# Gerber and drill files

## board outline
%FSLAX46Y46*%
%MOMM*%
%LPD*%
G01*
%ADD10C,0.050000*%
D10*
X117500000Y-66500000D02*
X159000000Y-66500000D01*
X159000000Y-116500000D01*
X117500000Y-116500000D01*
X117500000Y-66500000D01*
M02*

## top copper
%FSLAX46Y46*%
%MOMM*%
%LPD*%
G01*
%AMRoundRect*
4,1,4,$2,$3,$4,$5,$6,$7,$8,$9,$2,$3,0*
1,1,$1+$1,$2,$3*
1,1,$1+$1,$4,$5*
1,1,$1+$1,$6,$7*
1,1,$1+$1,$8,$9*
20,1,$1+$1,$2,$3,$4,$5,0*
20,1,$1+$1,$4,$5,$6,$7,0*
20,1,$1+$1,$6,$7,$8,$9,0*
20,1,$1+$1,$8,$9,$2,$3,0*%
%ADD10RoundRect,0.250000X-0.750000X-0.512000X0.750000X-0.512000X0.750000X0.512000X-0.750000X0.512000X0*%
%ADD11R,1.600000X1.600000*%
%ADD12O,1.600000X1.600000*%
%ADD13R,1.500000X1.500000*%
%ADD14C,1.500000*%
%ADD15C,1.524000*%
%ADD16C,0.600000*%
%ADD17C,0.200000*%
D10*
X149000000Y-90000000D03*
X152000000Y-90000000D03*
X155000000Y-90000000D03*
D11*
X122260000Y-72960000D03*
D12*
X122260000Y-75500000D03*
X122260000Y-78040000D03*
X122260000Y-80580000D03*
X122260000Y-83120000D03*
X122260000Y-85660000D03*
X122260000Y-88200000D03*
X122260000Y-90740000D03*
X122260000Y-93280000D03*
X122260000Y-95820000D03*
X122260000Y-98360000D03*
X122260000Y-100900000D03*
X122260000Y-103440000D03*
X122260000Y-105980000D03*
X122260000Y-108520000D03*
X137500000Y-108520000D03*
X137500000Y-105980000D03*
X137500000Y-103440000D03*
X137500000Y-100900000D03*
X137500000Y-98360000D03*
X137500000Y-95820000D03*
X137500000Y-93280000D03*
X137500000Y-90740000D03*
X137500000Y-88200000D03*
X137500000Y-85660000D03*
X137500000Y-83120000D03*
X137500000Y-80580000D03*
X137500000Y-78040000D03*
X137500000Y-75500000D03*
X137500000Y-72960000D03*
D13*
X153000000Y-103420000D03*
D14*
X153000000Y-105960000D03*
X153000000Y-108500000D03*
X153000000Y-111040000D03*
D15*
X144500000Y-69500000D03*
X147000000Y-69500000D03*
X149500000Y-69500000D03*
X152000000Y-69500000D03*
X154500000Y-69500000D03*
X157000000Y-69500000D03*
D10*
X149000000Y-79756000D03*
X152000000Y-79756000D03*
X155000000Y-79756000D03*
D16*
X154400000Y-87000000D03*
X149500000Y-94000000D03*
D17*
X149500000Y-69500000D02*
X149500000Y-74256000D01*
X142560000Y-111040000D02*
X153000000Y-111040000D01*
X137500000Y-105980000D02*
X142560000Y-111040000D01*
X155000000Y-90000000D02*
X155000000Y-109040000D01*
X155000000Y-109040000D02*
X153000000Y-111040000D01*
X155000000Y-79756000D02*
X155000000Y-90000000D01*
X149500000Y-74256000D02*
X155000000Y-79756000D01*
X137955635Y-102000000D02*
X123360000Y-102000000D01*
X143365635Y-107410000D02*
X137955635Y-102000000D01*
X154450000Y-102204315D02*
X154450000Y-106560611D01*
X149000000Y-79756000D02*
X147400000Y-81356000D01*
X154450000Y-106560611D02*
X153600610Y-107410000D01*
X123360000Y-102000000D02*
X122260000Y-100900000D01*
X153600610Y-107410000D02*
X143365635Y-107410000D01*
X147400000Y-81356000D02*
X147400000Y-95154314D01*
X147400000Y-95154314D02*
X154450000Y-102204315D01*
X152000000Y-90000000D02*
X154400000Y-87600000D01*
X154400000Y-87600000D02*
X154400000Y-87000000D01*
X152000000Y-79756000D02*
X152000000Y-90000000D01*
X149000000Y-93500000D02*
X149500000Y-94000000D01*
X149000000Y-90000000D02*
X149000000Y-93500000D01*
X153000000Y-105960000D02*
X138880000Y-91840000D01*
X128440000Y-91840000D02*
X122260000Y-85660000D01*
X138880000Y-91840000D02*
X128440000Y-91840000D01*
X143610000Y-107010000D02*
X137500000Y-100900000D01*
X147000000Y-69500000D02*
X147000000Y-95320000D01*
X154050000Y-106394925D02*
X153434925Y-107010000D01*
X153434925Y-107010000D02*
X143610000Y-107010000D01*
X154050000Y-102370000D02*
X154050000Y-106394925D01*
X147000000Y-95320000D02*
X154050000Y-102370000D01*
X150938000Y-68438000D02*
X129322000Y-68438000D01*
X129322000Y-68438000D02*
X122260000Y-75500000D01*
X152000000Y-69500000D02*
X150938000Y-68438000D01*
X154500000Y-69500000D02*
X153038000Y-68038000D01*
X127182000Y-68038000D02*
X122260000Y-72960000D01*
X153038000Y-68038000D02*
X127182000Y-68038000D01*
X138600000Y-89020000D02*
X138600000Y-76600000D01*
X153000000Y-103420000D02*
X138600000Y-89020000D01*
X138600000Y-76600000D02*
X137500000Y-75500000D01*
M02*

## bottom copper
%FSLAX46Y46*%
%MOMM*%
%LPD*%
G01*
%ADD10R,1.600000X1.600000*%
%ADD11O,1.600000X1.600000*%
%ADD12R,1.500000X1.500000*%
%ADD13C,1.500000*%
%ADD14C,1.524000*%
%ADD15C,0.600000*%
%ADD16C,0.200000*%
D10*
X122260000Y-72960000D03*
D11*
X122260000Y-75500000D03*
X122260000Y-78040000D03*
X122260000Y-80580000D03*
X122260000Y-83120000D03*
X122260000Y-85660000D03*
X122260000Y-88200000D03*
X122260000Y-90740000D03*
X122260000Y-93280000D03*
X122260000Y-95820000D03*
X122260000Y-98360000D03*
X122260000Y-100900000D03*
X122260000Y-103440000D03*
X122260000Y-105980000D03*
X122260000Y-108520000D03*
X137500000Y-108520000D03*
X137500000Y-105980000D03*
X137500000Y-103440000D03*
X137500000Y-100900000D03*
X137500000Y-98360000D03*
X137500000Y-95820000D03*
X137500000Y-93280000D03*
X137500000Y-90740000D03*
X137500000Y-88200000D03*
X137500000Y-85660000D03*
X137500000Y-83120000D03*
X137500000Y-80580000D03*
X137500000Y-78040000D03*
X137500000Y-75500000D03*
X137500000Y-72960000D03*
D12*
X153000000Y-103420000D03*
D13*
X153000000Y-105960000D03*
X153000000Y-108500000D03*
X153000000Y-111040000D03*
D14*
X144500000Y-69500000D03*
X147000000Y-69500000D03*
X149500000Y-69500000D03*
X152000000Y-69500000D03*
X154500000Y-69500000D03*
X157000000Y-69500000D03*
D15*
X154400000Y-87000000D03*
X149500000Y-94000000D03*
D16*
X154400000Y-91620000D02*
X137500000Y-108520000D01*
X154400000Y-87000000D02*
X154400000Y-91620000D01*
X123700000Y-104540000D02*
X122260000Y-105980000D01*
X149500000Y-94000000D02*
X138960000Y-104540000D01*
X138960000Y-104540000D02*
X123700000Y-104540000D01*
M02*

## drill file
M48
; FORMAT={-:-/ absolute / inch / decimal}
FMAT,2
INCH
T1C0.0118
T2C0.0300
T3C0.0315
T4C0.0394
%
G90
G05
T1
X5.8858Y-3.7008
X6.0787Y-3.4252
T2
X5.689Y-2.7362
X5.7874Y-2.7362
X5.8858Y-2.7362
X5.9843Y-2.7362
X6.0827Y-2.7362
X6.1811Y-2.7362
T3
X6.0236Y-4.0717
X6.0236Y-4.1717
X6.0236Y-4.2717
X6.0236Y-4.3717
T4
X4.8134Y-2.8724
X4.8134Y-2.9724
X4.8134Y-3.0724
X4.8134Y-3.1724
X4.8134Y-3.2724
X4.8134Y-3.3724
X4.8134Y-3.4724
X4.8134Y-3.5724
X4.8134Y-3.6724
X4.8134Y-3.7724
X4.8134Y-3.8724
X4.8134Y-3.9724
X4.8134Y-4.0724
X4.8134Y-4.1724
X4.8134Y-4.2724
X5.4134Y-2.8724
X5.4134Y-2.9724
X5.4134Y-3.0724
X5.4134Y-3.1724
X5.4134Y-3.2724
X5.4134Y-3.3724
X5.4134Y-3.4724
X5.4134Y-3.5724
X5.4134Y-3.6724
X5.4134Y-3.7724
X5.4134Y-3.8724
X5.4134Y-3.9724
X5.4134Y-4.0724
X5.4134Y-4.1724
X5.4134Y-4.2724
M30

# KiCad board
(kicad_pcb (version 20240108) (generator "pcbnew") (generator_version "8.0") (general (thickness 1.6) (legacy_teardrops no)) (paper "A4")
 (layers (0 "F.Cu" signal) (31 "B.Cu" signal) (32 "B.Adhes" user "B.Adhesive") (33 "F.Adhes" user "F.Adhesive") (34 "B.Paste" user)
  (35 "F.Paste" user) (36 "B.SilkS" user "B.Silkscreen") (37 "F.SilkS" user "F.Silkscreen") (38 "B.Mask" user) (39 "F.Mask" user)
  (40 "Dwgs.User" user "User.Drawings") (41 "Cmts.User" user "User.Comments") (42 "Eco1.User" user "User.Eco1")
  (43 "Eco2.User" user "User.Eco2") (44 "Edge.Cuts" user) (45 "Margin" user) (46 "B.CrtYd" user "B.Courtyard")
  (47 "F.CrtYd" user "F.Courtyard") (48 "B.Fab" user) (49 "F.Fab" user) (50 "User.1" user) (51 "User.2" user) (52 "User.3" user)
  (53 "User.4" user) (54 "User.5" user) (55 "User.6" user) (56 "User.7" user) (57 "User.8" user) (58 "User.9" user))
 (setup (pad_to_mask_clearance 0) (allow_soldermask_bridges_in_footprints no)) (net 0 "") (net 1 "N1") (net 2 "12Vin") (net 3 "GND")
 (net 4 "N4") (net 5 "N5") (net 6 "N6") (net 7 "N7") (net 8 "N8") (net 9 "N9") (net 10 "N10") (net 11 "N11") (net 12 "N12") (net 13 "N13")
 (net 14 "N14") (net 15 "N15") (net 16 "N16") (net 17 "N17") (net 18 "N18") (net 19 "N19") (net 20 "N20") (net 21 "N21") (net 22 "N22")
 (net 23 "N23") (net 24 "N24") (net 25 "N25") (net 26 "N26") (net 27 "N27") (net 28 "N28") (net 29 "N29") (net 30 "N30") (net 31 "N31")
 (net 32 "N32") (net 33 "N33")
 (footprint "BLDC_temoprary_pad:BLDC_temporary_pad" (layer "F.Cu") (at 152 95)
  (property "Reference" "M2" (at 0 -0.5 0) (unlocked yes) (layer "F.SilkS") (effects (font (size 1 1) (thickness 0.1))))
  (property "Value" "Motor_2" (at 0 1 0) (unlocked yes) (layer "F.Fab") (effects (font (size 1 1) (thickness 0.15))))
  (pad "1" smd roundrect (at -3 -5) (size 2 1.524) (layers "F.Cu" "F.Paste" "F.Mask") (roundrect_rratio 0.1640419948) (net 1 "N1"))
  (pad "2" smd roundrect (at 0 -5) (size 2 1.524) (layers "F.Cu" "F.Paste" "F.Mask") (roundrect_rratio 0.1640419948) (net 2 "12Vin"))
  (pad "3" smd roundrect (at 3 -5) (size 2 1.524) (layers "F.Cu" "F.Paste" "F.Mask") (roundrect_rratio 0.1640419948) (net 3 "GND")))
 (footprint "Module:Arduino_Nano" (layer "F.Cu") (at 122.26 72.96)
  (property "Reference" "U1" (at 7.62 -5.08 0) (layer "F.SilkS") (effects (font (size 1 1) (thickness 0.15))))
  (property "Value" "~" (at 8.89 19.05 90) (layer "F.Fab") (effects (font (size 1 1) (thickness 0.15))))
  (pad "1" thru_hole rect (at 0 0) (size 1.6 1.6) (drill 1) (layers "*.Cu" "*.Mask") (remove_unused_layers no) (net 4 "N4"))
  (pad "2" thru_hole oval (at 0 2.54) (size 1.6 1.6) (drill 1) (layers "*.Cu" "*.Mask") (remove_unused_layers no) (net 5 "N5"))
  (pad "3" thru_hole oval (at 0 5.08) (size 1.6 1.6) (drill 1) (layers "*.Cu" "*.Mask") (remove_unused_layers no) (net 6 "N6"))
  (pad "4" thru_hole oval (at 0 7.62) (size 1.6 1.6) (drill 1) (layers "*.Cu" "*.Mask") (remove_unused_layers no) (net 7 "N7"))
  (pad "5" thru_hole oval (at 0 10.16) (size 1.6 1.6) (drill 1) (layers "*.Cu" "*.Mask") (remove_unused_layers no) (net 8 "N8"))
  (pad "6" thru_hole oval (at 0 12.7) (size 1.6 1.6) (drill 1) (layers "*.Cu" "*.Mask") (remove_unused_layers no) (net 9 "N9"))
  (pad "7" thru_hole oval (at 0 15.24) (size 1.6 1.6) (drill 1) (layers "*.Cu" "*.Mask") (remove_unused_layers no) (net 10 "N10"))
  (pad "8" thru_hole oval (at 0 17.78) (size 1.6 1.6) (drill 1) (layers "*.Cu" "*.Mask") (remove_unused_layers no) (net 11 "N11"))
  (pad "9" thru_hole oval (at 0 20.32) (size 1.6 1.6) (drill 1) (layers "*.Cu" "*.Mask") (remove_unused_layers no) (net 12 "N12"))
  (pad "10" thru_hole oval (at 0 22.86) (size 1.6 1.6) (drill 1) (layers "*.Cu" "*.Mask") (remove_unused_layers no) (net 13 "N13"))
  (pad "11" thru_hole oval (at 0 25.4) (size 1.6 1.6) (drill 1) (layers "*.Cu" "*.Mask") (remove_unused_layers no) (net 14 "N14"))
  (pad "12" thru_hole oval (at 0 27.94) (size 1.6 1.6) (drill 1) (layers "*.Cu" "*.Mask") (remove_unused_layers no) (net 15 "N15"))
  (pad "13" thru_hole oval (at 0 30.48) (size 1.6 1.6) (drill 1) (layers "*.Cu" "*.Mask") (remove_unused_layers no) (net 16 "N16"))
  (pad "14" thru_hole oval (at 0 33.02) (size 1.6 1.6) (drill 1) (layers "*.Cu" "*.Mask") (remove_unused_layers no) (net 1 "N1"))
  (pad "15" thru_hole oval (at 0 35.56) (size 1.6 1.6) (drill 1) (layers "*.Cu" "*.Mask") (remove_unused_layers no) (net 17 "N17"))
  (pad "16" thru_hole oval (at 15.24 35.56) (size 1.6 1.6) (drill 1) (layers "*.Cu" "*.Mask") (remove_unused_layers no) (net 2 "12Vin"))
  (pad "17" thru_hole oval (at 15.24 33.02) (size 1.6 1.6) (drill 1) (layers "*.Cu" "*.Mask") (remove_unused_layers no) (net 3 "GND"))
  (pad "18" thru_hole oval (at 15.24 30.48) (size 1.6 1.6) (drill 1) (layers "*.Cu" "*.Mask") (remove_unused_layers no) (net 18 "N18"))
  (pad "19" thru_hole oval (at 15.24 27.94) (size 1.6 1.6) (drill 1) (layers "*.Cu" "*.Mask") (remove_unused_layers no) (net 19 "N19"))
  (pad "20" thru_hole oval (at 15.24 25.4) (size 1.6 1.6) (drill 1) (layers "*.Cu" "*.Mask") (remove_unused_layers no) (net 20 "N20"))
  (pad "21" thru_hole oval (at 15.24 22.86) (size 1.6 1.6) (drill 1) (layers "*.Cu" "*.Mask") (remove_unused_layers no) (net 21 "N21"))
  (pad "22" thru_hole oval (at 15.24 20.32) (size 1.6 1.6) (drill 1) (layers "*.Cu" "*.Mask") (remove_unused_layers no) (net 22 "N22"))
  (pad "23" thru_hole oval (at 15.24 17.78) (size 1.6 1.6) (drill 1) (layers "*.Cu" "*.Mask") (remove_unused_layers no) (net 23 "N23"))
  (pad "24" thru_hole oval (at 15.24 15.24) (size 1.6 1.6) (drill 1) (layers "*.Cu" "*.Mask") (remove_unused_layers no) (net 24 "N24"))
  (pad "25" thru_hole oval (at 15.24 12.7) (size 1.6 1.6) (drill 1) (layers "*.Cu" "*.Mask") (remove_unused_layers no) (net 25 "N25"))
  (pad "26" thru_hole oval (at 15.24 10.16) (size 1.6 1.6) (drill 1) (layers "*.Cu" "*.Mask") (remove_unused_layers no) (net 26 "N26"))
  (pad "27" thru_hole oval (at 15.24 7.62) (size 1.6 1.6) (drill 1) (layers "*.Cu" "*.Mask") (remove_unused_layers no) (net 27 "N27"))
  (pad "28" thru_hole oval (at 15.24 5.08) (size 1.6 1.6) (drill 1) (layers "*.Cu" "*.Mask") (remove_unused_layers no) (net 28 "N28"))
  (pad "29" thru_hole oval (at 15.24 2.54) (size 1.6 1.6) (drill 1) (layers "*.Cu" "*.Mask") (remove_unused_layers no) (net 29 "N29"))
  (pad "30" thru_hole oval (at 15.24 0) (size 1.6 1.6) (drill 1) (layers "*.Cu" "*.Mask") (remove_unused_layers no) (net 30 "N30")))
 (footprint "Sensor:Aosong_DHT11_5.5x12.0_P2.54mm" (layer "F.Cu") (at 153 103.42)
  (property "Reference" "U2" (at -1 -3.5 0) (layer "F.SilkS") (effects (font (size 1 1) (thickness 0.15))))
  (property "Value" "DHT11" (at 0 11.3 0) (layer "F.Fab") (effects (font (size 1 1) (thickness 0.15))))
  (pad "1" thru_hole rect (at 0 0) (size 1.5 1.5) (drill 0.8) (layers "*.Cu" "*.Mask") (remove_unused_layers no) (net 29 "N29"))
  (pad "2" thru_hole circle (at 0 2.54) (size 1.5 1.5) (drill 0.8) (layers "*.Cu" "*.Mask") (remove_unused_layers no) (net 9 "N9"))
  (pad "3" thru_hole circle (at 0 5.08) (size 1.5 1.5) (drill 0.8) (layers "*.Cu" "*.Mask") (remove_unused_layers no) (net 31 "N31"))
  (pad "4" thru_hole circle (at 0 7.62) (size 1.5 1.5) (drill 0.8) (layers "*.Cu" "*.Mask") (remove_unused_layers no) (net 3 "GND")))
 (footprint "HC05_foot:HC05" (layer "F.Cu") (at 148 76.5)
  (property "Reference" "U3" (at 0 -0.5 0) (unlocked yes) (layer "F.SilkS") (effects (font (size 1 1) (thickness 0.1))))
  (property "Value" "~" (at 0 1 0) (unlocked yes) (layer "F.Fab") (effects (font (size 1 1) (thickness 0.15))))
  (pad "1" thru_hole circle (at -3.5 -7) (size 1.524 1.524) (drill 0.762) (layers "*.Cu" "*.Mask") (remove_unused_layers no) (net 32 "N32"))
  (pad "2" thru_hole circle (at -1 -7) (size 1.524 1.524) (drill 0.762) (layers "*.Cu" "*.Mask") (remove_unused_layers no) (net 19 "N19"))
  (pad "3" thru_hole circle (at 1.5 -7) (size 1.524 1.524) (drill 0.762) (layers "*.Cu" "*.Mask") (remove_unused_layers no) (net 3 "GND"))
  (pad "4" thru_hole circle (at 4 -7) (size 1.524 1.524) (drill 0.762) (layers "*.Cu" "*.Mask") (remove_unused_layers no) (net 5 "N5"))
  (pad "5" thru_hole circle (at 6.5 -7) (size 1.524 1.524) (drill 0.762) (layers "*.Cu" "*.Mask") (remove_unused_layers no) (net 4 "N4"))
  (pad "6" thru_hole circle (at 9 -7) (size 1.524 1.524) (drill 0.762) (layers "*.Cu" "*.Mask") (remove_unused_layers no) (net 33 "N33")))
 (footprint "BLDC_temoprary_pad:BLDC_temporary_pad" (layer "F.Cu") (at 152 84.756)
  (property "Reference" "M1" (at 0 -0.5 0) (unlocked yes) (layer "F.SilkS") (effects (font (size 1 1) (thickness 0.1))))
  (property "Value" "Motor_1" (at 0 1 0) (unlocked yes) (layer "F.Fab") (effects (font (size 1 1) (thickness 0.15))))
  (pad "1" smd roundrect (at -3 -5) (size 2 1.524) (layers "F.Cu" "F.Paste" "F.Mask") (roundrect_rratio 0.1640419948) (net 15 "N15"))
  (pad "2" smd roundrect (at 0 -5) (size 2 1.524) (layers "F.Cu" "F.Paste" "F.Mask") (roundrect_rratio 0.1640419948) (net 2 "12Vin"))
  (pad "3" smd roundrect (at 3 -5) (size 2 1.524) (layers "F.Cu" "F.Paste" "F.Mask") (roundrect_rratio 0.1640419948) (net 3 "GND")))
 (gr_rect (start 117.5 66.5) (end 159 116.5) (stroke (width 0.05) (type default)) (fill none) (layer "Edge.Cuts"))
 (segment (start 149.5 69.5) (end 149.5 74.256) (width 0.2) (layer "F.Cu") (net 3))
 (segment (start 142.56 111.04) (end 153 111.04) (width 0.2) (layer "F.Cu") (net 3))
 (segment (start 137.5 105.98) (end 142.56 111.04) (width 0.2) (layer "F.Cu") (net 3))
 (segment (start 155 90) (end 155 109.04) (width 0.2) (layer "F.Cu") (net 3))
 (segment (start 155 109.04) (end 153 111.04) (width 0.2) (layer "F.Cu") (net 3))
 (segment (start 155 79.756) (end 155 90) (width 0.2) (layer "F.Cu") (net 3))
 (segment (start 149.5 74.256) (end 155 79.756) (width 0.2) (layer "F.Cu") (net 3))
 (segment (start 137.955635 102) (end 123.36 102) (width 0.2) (layer "F.Cu") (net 15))
 (segment (start 143.365635 107.41) (end 137.955635 102) (width 0.2) (layer "F.Cu") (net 15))
 (segment (start 154.45 102.204315) (end 154.45 106.560611) (width 0.2) (layer "F.Cu") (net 15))
 (segment (start 149 79.756) (end 147.4 81.356) (width 0.2) (layer "F.Cu") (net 15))
 (segment (start 154.45 106.560611) (end 153.60061 107.41) (width 0.2) (layer "F.Cu") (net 15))
 (segment (start 123.36 102) (end 122.26 100.9) (width 0.2) (layer "F.Cu") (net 15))
 (segment (start 153.60061 107.41) (end 143.365635 107.41) (width 0.2) (layer "F.Cu") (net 15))
 (segment (start 147.4 81.356) (end 147.4 95.154314) (width 0.2) (layer "F.Cu") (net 15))
 (segment (start 147.4 95.154314) (end 154.45 102.204315) (width 0.2) (layer "F.Cu") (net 15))
 (segment (start 152 90) (end 154.4 87.6) (width 0.2) (layer "F.Cu") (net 2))
 (segment (start 154.4 87.6) (end 154.4 87) (width 0.2) (layer "F.Cu") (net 2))
 (segment (start 152 79.756) (end 152 90) (width 0.2) (layer "F.Cu") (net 2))
 (via (at 154.4 87) (size 0.6) (drill 0.3) (layers "F.Cu" "B.Cu") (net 2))
 (segment (start 154.4 91.62) (end 137.5 108.52) (width 0.2) (layer "B.Cu") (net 2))
 (segment (start 154.4 87) (end 154.4 91.62) (width 0.2) (layer "B.Cu") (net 2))
 (segment (start 149 93.5) (end 149.5 94) (width 0.2) (layer "F.Cu") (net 1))
 (segment (start 149 90) (end 149 93.5) (width 0.2) (layer "F.Cu") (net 1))
 (via (at 149.5 94) (size 0.6) (drill 0.3) (layers "F.Cu" "B.Cu") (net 1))
 (segment (start 123.7 104.54) (end 122.26 105.98) (width 0.2) (layer "B.Cu") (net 1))
 (segment (start 149.5 94) (end 138.96 104.54) (width 0.2) (layer "B.Cu") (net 1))
 (segment (start 138.96 104.54) (end 123.7 104.54) (width 0.2) (layer "B.Cu") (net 1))
 (segment (start 153 105.96) (end 138.88 91.84) (width 0.2) (layer "F.Cu") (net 9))
 (segment (start 128.44 91.84) (end 122.26 85.66) (width 0.2) (layer "F.Cu") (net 9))
 (segment (start 138.88 91.84) (end 128.44 91.84) (width 0.2) (layer "F.Cu") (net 9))
 (segment (start 143.61 107.01) (end 137.5 100.9) (width 0.2) (layer "F.Cu") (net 19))
 (segment (start 147 69.5) (end 147 95.32) (width 0.2) (layer "F.Cu") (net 19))
 (segment (start 154.05 106.394925) (end 153.434925 107.01) (width 0.2) (layer "F.Cu") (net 19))
 (segment (start 153.434925 107.01) (end 143.61 107.01) (width 0.2) (layer "F.Cu") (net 19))
 (segment (start 154.05 102.37) (end 154.05 106.394925) (width 0.2) (layer "F.Cu") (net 19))
 (segment (start 147 95.32) (end 154.05 102.37) (width 0.2) (layer "F.Cu") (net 19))
 (segment (start 150.938 68.438) (end 129.322 68.438) (width 0.2) (layer "F.Cu") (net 5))
 (segment (start 129.322 68.438) (end 122.26 75.5) (width 0.2) (layer "F.Cu") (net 5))
 (segment (start 152 69.5) (end 150.938 68.438) (width 0.2) (layer "F.Cu") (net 5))
 (segment (start 154.5 69.5) (end 153.038 68.038) (width 0.2) (layer "F.Cu") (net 4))
 (segment (start 127.182 68.038) (end 122.26 72.96) (width 0.2) (layer "F.Cu") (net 4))
 (segment (start 153.038 68.038) (end 127.182 68.038) (width 0.2) (layer "F.Cu") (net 4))
 (segment (start 138.6 89.02) (end 138.6 76.6) (width 0.2) (layer "F.Cu") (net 29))
 (segment (start 153 103.42) (end 138.6 89.02) (width 0.2) (layer "F.Cu") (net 29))
 (segment (start 138.6 76.6) (end 137.5 75.5) (width 0.2) (layer "F.Cu") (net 29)))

